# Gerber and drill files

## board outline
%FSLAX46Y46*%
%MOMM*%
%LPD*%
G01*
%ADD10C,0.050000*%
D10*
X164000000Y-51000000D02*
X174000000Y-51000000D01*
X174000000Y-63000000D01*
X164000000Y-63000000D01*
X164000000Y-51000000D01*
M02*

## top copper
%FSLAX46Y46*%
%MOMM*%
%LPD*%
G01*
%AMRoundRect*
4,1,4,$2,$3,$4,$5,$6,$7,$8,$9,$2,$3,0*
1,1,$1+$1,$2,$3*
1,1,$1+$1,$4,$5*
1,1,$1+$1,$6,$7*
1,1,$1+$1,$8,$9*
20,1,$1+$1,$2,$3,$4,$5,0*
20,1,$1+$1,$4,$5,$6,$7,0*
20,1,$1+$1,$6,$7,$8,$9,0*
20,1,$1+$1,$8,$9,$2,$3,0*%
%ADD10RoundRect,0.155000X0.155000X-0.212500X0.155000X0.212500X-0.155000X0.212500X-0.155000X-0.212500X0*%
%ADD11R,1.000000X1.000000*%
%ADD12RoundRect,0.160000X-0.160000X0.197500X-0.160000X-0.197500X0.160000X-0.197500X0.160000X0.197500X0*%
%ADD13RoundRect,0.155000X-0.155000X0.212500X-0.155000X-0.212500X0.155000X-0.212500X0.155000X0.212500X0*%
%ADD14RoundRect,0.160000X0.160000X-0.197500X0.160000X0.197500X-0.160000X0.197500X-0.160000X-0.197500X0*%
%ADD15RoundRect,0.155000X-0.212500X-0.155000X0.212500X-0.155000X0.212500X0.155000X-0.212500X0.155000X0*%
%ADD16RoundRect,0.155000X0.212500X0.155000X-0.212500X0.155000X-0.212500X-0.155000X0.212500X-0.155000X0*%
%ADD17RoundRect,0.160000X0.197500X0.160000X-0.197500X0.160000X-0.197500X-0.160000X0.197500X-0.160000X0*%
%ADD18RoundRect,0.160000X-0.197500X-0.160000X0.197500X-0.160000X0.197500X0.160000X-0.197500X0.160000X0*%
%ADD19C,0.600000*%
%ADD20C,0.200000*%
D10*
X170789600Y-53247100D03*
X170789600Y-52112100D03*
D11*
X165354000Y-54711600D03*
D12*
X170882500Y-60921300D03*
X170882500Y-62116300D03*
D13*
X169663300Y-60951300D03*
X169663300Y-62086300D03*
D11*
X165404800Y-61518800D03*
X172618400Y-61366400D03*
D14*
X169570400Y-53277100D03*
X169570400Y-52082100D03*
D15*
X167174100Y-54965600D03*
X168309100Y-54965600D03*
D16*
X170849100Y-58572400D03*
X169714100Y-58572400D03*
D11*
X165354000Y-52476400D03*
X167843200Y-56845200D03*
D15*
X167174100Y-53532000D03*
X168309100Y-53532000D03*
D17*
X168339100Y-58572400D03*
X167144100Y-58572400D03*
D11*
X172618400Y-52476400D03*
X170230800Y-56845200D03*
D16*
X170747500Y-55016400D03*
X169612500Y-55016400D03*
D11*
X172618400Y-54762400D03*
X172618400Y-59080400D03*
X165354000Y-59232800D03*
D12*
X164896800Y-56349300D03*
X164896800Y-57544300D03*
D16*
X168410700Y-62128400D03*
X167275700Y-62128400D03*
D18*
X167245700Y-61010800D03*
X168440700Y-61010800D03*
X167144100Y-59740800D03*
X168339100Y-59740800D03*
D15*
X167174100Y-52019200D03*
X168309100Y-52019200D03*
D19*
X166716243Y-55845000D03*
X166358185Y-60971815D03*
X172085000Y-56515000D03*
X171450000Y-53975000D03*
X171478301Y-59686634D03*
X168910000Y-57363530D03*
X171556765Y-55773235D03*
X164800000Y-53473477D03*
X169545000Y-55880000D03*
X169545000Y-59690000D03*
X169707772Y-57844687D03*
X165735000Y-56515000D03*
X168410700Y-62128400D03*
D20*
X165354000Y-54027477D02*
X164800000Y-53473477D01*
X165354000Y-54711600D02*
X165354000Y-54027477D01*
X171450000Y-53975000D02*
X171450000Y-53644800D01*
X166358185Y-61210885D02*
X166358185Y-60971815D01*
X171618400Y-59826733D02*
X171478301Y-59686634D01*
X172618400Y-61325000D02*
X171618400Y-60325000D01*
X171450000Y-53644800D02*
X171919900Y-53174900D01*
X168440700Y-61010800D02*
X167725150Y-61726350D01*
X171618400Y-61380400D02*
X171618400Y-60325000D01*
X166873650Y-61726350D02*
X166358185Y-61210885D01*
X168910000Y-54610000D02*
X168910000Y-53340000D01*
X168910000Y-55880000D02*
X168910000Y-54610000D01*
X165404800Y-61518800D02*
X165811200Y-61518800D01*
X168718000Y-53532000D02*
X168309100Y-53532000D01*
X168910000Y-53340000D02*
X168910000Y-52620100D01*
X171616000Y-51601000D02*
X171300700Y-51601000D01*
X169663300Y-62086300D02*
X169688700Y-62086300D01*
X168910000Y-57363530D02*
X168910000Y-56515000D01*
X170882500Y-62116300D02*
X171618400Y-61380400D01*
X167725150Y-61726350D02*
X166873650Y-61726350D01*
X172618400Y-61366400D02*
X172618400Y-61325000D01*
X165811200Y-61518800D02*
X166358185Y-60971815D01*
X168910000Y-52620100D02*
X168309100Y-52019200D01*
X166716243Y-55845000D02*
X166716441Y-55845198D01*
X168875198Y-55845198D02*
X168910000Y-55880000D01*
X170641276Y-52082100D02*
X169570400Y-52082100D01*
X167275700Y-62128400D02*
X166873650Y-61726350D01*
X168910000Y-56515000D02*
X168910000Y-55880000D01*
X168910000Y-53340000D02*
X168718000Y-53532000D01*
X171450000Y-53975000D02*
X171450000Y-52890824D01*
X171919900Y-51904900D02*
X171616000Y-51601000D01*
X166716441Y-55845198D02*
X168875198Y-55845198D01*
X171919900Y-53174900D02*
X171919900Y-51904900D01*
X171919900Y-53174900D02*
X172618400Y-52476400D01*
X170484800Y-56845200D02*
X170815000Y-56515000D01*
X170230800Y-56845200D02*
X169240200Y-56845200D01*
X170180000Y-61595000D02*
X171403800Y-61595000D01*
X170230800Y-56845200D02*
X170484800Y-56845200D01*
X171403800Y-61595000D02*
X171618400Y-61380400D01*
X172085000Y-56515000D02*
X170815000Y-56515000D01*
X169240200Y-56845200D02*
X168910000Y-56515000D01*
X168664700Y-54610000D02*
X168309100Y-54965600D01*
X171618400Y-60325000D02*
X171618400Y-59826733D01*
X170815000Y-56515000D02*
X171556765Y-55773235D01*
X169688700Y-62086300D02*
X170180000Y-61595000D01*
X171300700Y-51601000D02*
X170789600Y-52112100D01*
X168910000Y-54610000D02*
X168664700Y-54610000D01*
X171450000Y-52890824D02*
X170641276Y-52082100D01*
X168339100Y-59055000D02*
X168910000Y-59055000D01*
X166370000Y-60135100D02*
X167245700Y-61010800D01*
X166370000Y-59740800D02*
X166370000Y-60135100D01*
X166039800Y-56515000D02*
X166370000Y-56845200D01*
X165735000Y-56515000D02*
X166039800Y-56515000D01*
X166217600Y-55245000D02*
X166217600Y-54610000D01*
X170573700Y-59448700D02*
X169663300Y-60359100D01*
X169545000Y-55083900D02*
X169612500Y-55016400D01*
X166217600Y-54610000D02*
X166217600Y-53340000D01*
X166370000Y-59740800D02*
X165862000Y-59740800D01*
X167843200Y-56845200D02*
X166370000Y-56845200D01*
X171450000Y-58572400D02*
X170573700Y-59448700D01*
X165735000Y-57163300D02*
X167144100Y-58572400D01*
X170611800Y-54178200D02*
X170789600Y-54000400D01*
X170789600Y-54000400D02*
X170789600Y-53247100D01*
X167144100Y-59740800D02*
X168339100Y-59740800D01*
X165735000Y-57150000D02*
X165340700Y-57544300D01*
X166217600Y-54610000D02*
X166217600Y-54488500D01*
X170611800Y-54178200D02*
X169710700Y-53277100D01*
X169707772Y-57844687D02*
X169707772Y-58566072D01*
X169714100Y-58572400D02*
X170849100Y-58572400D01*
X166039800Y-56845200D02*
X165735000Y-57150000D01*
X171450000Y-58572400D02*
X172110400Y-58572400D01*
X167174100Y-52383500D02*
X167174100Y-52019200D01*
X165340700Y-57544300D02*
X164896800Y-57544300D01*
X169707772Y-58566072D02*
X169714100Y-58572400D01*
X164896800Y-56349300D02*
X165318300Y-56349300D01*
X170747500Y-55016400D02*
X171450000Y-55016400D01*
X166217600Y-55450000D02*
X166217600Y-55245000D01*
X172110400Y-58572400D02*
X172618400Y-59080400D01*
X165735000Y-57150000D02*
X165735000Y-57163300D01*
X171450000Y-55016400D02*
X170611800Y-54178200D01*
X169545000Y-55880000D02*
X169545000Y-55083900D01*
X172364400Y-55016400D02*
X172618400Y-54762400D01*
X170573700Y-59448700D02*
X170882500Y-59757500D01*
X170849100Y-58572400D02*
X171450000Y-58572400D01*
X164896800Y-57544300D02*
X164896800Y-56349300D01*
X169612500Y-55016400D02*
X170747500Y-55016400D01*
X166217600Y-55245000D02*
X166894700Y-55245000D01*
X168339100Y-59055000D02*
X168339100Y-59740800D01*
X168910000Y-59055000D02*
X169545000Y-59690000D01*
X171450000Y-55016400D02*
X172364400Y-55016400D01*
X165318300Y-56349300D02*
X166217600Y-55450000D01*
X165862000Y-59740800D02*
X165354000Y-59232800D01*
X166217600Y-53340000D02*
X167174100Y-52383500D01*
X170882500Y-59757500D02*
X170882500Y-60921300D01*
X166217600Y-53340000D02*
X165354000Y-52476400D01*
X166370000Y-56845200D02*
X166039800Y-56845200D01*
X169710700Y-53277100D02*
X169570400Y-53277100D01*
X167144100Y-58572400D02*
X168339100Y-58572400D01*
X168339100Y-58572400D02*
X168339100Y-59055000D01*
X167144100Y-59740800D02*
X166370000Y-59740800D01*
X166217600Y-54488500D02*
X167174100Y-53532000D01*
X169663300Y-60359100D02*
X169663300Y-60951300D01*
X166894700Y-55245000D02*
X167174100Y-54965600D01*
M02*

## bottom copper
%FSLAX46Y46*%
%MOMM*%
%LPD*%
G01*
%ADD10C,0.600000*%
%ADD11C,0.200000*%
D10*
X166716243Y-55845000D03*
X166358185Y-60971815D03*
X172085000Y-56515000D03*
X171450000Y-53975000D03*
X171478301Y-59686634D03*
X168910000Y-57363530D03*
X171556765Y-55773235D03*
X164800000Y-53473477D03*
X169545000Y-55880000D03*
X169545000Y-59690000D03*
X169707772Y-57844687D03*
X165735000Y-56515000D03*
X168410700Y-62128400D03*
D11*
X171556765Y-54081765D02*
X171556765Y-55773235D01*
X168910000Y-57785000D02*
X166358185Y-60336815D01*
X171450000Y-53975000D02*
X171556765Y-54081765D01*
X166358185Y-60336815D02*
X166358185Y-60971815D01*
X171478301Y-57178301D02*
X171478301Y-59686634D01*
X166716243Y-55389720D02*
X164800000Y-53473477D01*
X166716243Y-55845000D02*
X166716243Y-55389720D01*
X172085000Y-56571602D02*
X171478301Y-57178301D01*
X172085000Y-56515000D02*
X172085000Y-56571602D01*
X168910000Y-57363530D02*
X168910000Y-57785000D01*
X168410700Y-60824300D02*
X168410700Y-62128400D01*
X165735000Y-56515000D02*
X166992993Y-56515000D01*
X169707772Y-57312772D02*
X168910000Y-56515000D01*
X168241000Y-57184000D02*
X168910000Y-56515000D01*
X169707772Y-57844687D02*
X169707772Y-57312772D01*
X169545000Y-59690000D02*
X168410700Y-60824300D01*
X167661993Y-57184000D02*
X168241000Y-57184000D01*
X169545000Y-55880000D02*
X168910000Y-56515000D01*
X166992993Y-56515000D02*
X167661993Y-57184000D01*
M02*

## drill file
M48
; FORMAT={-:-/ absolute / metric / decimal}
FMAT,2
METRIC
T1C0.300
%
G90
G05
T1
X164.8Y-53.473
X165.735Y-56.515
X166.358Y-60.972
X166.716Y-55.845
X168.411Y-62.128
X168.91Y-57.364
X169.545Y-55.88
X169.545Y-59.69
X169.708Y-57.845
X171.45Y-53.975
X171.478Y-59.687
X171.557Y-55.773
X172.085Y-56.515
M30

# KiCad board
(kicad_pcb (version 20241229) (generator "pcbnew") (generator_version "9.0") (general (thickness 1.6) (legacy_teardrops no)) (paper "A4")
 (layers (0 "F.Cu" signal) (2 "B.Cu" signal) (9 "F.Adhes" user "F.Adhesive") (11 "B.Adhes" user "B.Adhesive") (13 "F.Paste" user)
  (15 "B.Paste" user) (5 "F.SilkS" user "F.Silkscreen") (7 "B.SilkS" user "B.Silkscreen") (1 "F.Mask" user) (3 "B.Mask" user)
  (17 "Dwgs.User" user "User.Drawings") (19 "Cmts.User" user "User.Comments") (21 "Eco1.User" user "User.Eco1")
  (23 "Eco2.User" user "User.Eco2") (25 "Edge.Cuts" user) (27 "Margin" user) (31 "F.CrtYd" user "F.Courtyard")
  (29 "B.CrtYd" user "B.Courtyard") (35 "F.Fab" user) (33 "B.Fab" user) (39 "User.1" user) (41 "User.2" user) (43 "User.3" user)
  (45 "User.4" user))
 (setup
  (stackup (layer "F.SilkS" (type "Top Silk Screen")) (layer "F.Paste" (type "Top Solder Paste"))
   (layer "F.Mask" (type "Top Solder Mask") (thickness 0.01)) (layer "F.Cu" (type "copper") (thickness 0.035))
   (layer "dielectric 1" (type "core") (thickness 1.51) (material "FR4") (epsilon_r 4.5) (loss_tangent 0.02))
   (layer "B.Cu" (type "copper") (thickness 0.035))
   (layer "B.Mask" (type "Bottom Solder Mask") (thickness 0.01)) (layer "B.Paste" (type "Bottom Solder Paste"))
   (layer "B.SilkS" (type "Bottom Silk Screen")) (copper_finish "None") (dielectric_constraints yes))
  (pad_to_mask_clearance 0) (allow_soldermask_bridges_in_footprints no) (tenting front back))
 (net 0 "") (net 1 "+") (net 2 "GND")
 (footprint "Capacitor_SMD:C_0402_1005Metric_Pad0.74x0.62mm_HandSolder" (layer "F.Cu") (at 170.7896 52.6796 90)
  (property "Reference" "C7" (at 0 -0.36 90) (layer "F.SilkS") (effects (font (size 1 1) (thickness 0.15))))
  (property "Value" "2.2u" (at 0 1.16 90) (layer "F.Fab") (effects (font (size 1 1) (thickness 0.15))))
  (pad "1" smd roundrect (at -0.5675 0 90) (size 0.735 0.62) (layers "F.Cu" "F.Mask" "F.Paste") (roundrect_rratio 0.25) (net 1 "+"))
  (pad "2" smd roundrect (at 0.5675 0 90) (size 0.735 0.62) (layers "F.Cu" "F.Mask" "F.Paste") (roundrect_rratio 0.25) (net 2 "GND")))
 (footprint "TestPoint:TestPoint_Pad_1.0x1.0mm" (layer "F.Cu") (at 165.354 54.7116)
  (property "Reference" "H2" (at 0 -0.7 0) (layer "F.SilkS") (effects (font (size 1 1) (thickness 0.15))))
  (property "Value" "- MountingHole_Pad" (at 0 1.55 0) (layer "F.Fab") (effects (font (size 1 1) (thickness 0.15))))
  (pad "1" smd rect (at 0 0) (size 1 1) (layers "F.Cu" "F.Mask")))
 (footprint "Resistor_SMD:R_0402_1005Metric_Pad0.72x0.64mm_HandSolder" (layer "F.Cu") (at 170.8825 61.5188 -90)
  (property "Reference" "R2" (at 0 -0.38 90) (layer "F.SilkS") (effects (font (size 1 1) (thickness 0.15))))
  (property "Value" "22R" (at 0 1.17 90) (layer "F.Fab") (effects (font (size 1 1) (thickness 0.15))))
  (pad "1" smd roundrect (at -0.5975 0 270) (size 0.715 0.64) (layers "F.Cu" "F.Mask" "F.Paste") (roundrect_rratio 0.25) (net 1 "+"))
  (pad "2" smd roundrect (at 0.5975 0 270) (size 0.715 0.64) (layers "F.Cu" "F.Mask" "F.Paste") (roundrect_rratio 0.25) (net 2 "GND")))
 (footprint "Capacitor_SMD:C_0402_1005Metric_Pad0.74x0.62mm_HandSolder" (layer "F.Cu") (at 169.6633 61.5188 -90)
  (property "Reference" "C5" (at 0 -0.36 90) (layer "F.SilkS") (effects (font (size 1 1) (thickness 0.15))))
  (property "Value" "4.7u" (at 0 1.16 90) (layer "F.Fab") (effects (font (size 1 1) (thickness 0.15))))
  (pad "1" smd roundrect (at -0.5675 0 270) (size 0.735 0.62) (layers "F.Cu" "F.Mask" "F.Paste") (roundrect_rratio 0.25) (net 1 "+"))
  (pad "2" smd roundrect (at 0.5675 0 270) (size 0.735 0.62) (layers "F.Cu" "F.Mask" "F.Paste") (roundrect_rratio 0.25) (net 2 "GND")))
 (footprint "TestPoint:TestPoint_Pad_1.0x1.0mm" (layer "F.Cu") (at 165.4048 61.5188)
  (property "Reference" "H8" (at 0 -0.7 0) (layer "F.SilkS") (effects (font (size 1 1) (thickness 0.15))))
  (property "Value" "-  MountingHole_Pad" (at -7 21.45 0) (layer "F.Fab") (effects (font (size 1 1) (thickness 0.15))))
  (pad "1" smd rect (at 0 0) (size 1 1) (layers "F.Cu" "F.Mask")))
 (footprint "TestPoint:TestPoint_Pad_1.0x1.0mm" (layer "F.Cu") (at 172.6184 61.3664)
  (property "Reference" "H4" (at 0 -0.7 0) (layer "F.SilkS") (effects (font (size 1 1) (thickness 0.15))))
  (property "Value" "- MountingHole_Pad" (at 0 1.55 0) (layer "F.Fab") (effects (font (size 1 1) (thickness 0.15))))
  (pad "1" smd rect (at 0 0) (size 1 1) (layers "F.Cu" "F.Mask")))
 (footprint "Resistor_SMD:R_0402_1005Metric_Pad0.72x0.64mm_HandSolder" (layer "F.Cu") (at 169.5704 52.6796 90)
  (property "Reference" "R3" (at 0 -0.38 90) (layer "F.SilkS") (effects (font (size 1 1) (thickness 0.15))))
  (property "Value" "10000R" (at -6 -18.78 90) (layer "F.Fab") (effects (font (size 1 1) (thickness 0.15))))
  (pad "1" smd roundrect (at -0.5975 0 90) (size 0.715 0.64) (layers "F.Cu" "F.Mask" "F.Paste") (roundrect_rratio 0.25) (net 1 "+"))
  (pad "2" smd roundrect (at 0.5975 0 90) (size 0.715 0.64) (layers "F.Cu" "F.Mask" "F.Paste") (roundrect_rratio 0.25) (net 2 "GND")))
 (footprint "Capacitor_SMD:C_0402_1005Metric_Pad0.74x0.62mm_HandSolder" (layer "F.Cu") (at 167.7416 54.9656)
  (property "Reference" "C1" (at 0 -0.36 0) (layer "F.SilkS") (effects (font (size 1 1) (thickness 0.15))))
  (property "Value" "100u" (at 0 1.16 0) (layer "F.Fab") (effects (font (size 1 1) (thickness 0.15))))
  (pad "1" smd roundrect (at -0.5675 0) (size 0.735 0.62) (layers "F.Cu" "F.Mask" "F.Paste") (roundrect_rratio 0.25) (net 1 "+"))
  (pad "2" smd roundrect (at 0.5675 0) (size 0.735 0.62) (layers "F.Cu" "F.Mask" "F.Paste") (roundrect_rratio 0.25) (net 2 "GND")))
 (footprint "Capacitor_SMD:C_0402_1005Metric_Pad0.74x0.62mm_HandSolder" (layer "F.Cu") (at 170.2816 58.5724 180)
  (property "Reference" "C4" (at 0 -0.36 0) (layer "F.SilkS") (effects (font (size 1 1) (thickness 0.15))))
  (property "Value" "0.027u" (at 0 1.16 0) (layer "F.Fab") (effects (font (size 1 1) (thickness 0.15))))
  (pad "1" smd roundrect (at -0.5675 0 180) (size 0.735 0.62) (layers "F.Cu" "F.Mask" "F.Paste") (roundrect_rratio 0.25) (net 1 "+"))
  (pad "2" smd roundrect (at 0.5675 0 180) (size 0.735 0.62) (layers "F.Cu" "F.Mask" "F.Paste") (roundrect_rratio 0.25) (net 1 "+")))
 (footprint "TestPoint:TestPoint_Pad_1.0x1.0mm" (layer "F.Cu") (at 165.354 52.4764)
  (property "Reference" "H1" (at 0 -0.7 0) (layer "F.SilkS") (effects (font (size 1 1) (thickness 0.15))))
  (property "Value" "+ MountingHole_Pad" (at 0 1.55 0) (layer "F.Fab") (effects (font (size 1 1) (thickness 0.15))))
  (pad "1" smd rect (at 0 0) (size 1 1) (layers "F.Cu" "F.Mask") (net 1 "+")))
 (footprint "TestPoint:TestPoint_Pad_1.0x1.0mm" (layer "F.Cu") (at 167.8432 56.8452)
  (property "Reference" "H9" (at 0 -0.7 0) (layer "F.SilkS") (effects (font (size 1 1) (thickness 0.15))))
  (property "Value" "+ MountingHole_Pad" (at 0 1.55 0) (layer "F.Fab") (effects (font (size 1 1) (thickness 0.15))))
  (pad "1" smd rect (at 0 0) (size 1 1) (layers "F.Cu" "F.Mask") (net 1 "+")))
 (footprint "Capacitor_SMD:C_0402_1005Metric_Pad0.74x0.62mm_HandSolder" (layer "F.Cu") (at 167.7416 53.532)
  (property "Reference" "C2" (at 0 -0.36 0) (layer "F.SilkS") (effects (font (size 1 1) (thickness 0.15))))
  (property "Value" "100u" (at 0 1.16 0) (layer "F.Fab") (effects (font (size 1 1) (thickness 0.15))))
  (pad "1" smd roundrect (at -0.5675 0) (size 0.735 0.62) (layers "F.Cu" "F.Mask" "F.Paste") (roundrect_rratio 0.25) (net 1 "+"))
  (pad "2" smd roundrect (at 0.5675 0) (size 0.735 0.62) (layers "F.Cu" "F.Mask" "F.Paste") (roundrect_rratio 0.25) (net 2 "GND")))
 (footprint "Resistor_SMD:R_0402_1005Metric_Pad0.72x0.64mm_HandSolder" (layer "F.Cu") (at 167.7416 58.5724 180)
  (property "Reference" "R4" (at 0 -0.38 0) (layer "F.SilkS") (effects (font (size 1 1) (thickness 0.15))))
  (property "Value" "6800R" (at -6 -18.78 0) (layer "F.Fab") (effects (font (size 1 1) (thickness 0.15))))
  (pad "1" smd roundrect (at -0.5975 0 180) (size 0.715 0.64) (layers "F.Cu" "F.Mask" "F.Paste") (roundrect_rratio 0.25) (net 1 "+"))
  (pad "2" smd roundrect (at 0.5975 0 180) (size 0.715 0.64) (layers "F.Cu" "F.Mask" "F.Paste") (roundrect_rratio 0.25) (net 1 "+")))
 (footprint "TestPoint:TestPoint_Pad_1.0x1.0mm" (layer "F.Cu") (at 172.6184 52.4764)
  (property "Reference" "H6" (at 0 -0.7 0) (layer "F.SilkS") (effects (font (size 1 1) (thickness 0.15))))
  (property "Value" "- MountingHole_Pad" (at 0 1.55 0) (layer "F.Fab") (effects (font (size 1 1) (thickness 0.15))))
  (pad "1" smd rect (at 0 0) (size 1 1) (layers "F.Cu" "F.Mask")))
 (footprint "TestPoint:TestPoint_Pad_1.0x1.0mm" (layer "F.Cu") (at 170.2308 56.8452)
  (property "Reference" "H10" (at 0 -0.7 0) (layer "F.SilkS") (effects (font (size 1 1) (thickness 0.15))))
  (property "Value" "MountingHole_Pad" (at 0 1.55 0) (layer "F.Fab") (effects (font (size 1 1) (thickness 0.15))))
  (pad "1" smd rect (at 0 0) (size 1 1) (layers "F.Cu" "F.Mask")))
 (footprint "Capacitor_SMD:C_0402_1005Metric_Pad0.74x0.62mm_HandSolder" (layer "F.Cu") (at 170.18 55.0164 180)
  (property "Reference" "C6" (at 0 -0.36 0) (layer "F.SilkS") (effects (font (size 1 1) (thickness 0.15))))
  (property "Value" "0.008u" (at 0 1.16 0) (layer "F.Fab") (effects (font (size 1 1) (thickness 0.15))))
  (pad "1" smd roundrect (at -0.5675 0 180) (size 0.735 0.62) (layers "F.Cu" "F.Mask" "F.Paste") (roundrect_rratio 0.25) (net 1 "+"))
  (pad "2" smd roundrect (at 0.5675 0 180) (size 0.735 0.62) (layers "F.Cu" "F.Mask" "F.Paste") (roundrect_rratio 0.25) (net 1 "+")))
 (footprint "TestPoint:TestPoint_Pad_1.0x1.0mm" (layer "F.Cu") (at 172.6184 54.7624)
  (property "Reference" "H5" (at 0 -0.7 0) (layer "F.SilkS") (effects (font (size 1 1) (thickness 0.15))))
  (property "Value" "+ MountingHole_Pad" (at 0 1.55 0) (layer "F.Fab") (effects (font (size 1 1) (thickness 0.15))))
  (pad "1" smd rect (at 0 0) (size 1 1) (layers "F.Cu" "F.Mask") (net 1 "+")))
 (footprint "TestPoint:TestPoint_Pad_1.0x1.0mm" (layer "F.Cu") (at 172.6184 59.0804)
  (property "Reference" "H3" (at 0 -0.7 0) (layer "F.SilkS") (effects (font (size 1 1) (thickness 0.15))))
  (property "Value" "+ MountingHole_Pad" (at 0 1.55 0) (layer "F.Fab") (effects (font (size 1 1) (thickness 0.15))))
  (pad "1" smd rect (at 0 0) (size 1 1) (layers "F.Cu" "F.Mask") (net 1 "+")))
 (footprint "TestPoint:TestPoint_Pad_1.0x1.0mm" (layer "F.Cu") (at 165.354 59.2328)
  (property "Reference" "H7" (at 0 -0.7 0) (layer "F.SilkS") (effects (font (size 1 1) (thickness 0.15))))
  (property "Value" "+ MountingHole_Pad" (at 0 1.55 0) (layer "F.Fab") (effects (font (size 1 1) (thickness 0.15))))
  (pad "1" smd rect (at 0 0) (size 1 1) (layers "F.Cu" "F.Mask") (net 1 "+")))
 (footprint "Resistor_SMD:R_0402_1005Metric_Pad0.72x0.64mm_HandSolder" (layer "F.Cu") (at 164.8968 56.9468 -90)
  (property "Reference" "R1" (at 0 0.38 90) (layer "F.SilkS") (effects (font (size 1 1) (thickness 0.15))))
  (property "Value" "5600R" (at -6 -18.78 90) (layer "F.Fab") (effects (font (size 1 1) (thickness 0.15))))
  (pad "1" smd roundrect (at -0.5975 0 270) (size 0.715 0.64) (layers "F.Cu" "F.Mask" "F.Paste") (roundrect_rratio 0.25) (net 1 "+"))
  (pad "2" smd roundrect (at 0.5975 0 270) (size 0.715 0.64) (layers "F.Cu" "F.Mask" "F.Paste") (roundrect_rratio 0.25) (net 1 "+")))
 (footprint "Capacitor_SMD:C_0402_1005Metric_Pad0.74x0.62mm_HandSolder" (layer "F.Cu") (at 167.8432 62.1284 180)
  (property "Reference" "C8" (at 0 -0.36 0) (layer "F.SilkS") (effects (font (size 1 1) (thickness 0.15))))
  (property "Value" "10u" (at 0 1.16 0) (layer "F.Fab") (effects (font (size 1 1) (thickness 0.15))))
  (pad "1" smd roundrect (at -0.5675 0 180) (size 0.735 0.62) (layers "F.Cu" "F.Mask" "F.Paste") (roundrect_rratio 0.25) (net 1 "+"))
  (pad "2" smd roundrect (at 0.5675 0 180) (size 0.735 0.62) (layers "F.Cu" "F.Mask" "F.Paste") (roundrect_rratio 0.25) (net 2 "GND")))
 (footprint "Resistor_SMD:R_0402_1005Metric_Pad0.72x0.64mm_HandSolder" (layer "F.Cu") (at 167.8432 61.0108)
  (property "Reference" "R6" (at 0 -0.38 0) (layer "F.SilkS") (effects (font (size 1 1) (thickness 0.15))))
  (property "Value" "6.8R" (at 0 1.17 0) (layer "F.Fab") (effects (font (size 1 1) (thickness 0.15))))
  (pad "1" smd roundrect (at -0.5975 0) (size 0.715 0.64) (layers "F.Cu" "F.Mask" "F.Paste") (roundrect_rratio 0.25) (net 1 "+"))
  (pad "2" smd roundrect (at 0.5975 0) (size 0.715 0.64) (layers "F.Cu" "F.Mask" "F.Paste") (roundrect_rratio 0.25) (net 2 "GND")))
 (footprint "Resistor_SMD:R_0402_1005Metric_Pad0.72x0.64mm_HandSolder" (layer "F.Cu") (at 167.7416 59.7408)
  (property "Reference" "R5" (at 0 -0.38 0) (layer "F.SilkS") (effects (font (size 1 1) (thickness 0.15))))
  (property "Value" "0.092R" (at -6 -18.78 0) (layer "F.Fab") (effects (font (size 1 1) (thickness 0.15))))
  (pad "1" smd roundrect (at -0.5975 0) (size 0.715 0.64) (layers "F.Cu" "F.Mask" "F.Paste") (roundrect_rratio 0.25) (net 1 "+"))
  (pad "2" smd roundrect (at 0.5975 0) (size 0.715 0.64) (layers "F.Cu" "F.Mask" "F.Paste") (roundrect_rratio 0.25) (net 1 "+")))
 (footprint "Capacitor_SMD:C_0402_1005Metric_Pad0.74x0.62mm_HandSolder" (layer "F.Cu") (at 167.7416 52.0192)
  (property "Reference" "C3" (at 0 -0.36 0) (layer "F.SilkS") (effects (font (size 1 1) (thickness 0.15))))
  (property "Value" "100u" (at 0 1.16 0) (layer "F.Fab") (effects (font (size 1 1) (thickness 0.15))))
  (pad "1" smd roundrect (at -0.5675 0) (size 0.735 0.62) (layers "F.Cu" "F.Mask" "F.Paste") (roundrect_rratio 0.25) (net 1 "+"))
  (pad "2" smd roundrect (at 0.5675 0) (size 0.735 0.62) (layers "F.Cu" "F.Mask" "F.Paste") (roundrect_rratio 0.25) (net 2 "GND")))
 (gr_rect (start 164 51) (end 174 63) (stroke (width 0.05) (type default)) (fill no) (layer "Edge.Cuts"))
 (segment (start 165.354 54.027477) (end 164.8 53.473477) (width 0.2) (layer "F.Cu") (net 2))
 (segment (start 165.354 54.7116) (end 165.354 54.027477) (width 0.2) (layer "F.Cu") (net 2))
 (segment (start 171.45 53.975) (end 171.45 53.6448) (width 0.2) (layer "F.Cu") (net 2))
 (segment (start 166.358185 61.210885) (end 166.358185 60.971815) (width 0.2) (layer "F.Cu") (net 2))
 (segment (start 171.6184 59.826733) (end 171.478301 59.686634) (width 0.2) (layer "F.Cu") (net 2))
 (segment (start 172.6184 61.325) (end 171.6184 60.325) (width 0.2) (layer "F.Cu") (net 2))
 (segment (start 171.45 53.6448) (end 171.9199 53.1749) (width 0.2) (layer "F.Cu") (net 2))
 (segment (start 168.4407 61.0108) (end 167.72515 61.72635) (width 0.2) (layer "F.Cu") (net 2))
 (segment (start 171.6184 61.3804) (end 171.6184 60.325) (width 0.2) (layer "F.Cu") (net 2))
 (segment (start 166.87365 61.72635) (end 166.358185 61.210885) (width 0.2) (layer "F.Cu") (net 2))
 (segment (start 168.91 54.61) (end 168.91 53.34) (width 0.2) (layer "F.Cu") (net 2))
 (segment (start 168.91 55.88) (end 168.91 54.61) (width 0.2) (layer "F.Cu") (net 2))
 (segment (start 165.4048 61.5188) (end 165.8112 61.5188) (width 0.2) (layer "F.Cu") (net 2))
 (segment (start 168.718 53.532) (end 168.3091 53.532) (width 0.2) (layer "F.Cu") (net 2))
 (segment (start 168.91 53.34) (end 168.91 52.6201) (width 0.2) (layer "F.Cu") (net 2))
 (segment (start 171.616 51.601) (end 171.3007 51.601) (width 0.2) (layer "F.Cu") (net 2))
 (segment (start 169.6633 62.0863) (end 169.6887 62.0863) (width 0.2) (layer "F.Cu") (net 2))
 (segment (start 168.91 57.36353) (end 168.91 56.515) (width 0.2) (layer "F.Cu") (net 2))
 (segment (start 170.8825 62.1163) (end 171.6184 61.3804) (width 0.2) (layer "F.Cu") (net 2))
 (segment (start 167.72515 61.72635) (end 166.87365 61.72635) (width 0.2) (layer "F.Cu") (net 2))
 (segment (start 172.6184 61.3664) (end 172.6184 61.325) (width 0.2) (layer "F.Cu") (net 2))
 (segment (start 165.8112 61.5188) (end 166.358185 60.971815) (width 0.2) (layer "F.Cu") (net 2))
 (segment (start 168.91 52.6201) (end 168.3091 52.0192) (width 0.2) (layer "F.Cu") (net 2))
 (segment (start 166.716243 55.845) (end 166.716441 55.845198) (width 0.2) (layer "F.Cu") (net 2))
 (segment (start 168.875198 55.845198) (end 168.91 55.88) (width 0.2) (layer "F.Cu") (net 2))
 (segment (start 170.641276 52.0821) (end 169.5704 52.0821) (width 0.2) (layer "F.Cu") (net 2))
 (segment (start 167.2757 62.1284) (end 166.87365 61.72635) (width 0.2) (layer "F.Cu") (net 2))
 (segment (start 168.91 56.515) (end 168.91 55.88) (width 0.2) (layer "F.Cu") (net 2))
 (segment (start 168.91 53.34) (end 168.718 53.532) (width 0.2) (layer "F.Cu") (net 2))
 (segment (start 171.45 53.975) (end 171.45 52.890824) (width 0.2) (layer "F.Cu") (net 2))
 (segment (start 171.9199 51.9049) (end 171.616 51.601) (width 0.2) (layer "F.Cu") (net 2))
 (segment (start 166.716441 55.845198) (end 168.875198 55.845198) (width 0.2) (layer "F.Cu") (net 2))
 (segment (start 171.9199 53.1749) (end 171.9199 51.9049) (width 0.2) (layer "F.Cu") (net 2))
 (segment (start 171.9199 53.1749) (end 172.6184 52.4764) (width 0.2) (layer "F.Cu") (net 2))
 (segment (start 170.4848 56.8452) (end 170.815 56.515) (width 0.2) (layer "F.Cu") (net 2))
 (segment (start 170.2308 56.8452) (end 169.2402 56.8452) (width 0.2) (layer "F.Cu") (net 2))
 (segment (start 170.18 61.595) (end 171.4038 61.595) (width 0.2) (layer "F.Cu") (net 2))
 (segment (start 170.2308 56.8452) (end 170.4848 56.8452) (width 0.2) (layer "F.Cu") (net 2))
 (segment (start 171.4038 61.595) (end 171.6184 61.3804) (width 0.2) (layer "F.Cu") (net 2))
 (segment (start 172.085 56.515) (end 170.815 56.515) (width 0.2) (layer "F.Cu") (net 2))
 (segment (start 169.2402 56.8452) (end 168.91 56.515) (width 0.2) (layer "F.Cu") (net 2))
 (segment (start 168.6647 54.61) (end 168.3091 54.9656) (width 0.2) (layer "F.Cu") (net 2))
 (segment (start 171.6184 60.325) (end 171.6184 59.826733) (width 0.2) (layer "F.Cu") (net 2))
 (segment (start 170.815 56.515) (end 171.556765 55.773235) (width 0.2) (layer "F.Cu") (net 2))
 (segment (start 169.6887 62.0863) (end 170.18 61.595) (width 0.2) (layer "F.Cu") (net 2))
 (segment (start 171.3007 51.601) (end 170.7896 52.1121) (width 0.2) (layer "F.Cu") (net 2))
 (segment (start 168.91 54.61) (end 168.6647 54.61) (width 0.2) (layer "F.Cu") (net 2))
 (segment (start 171.45 52.890824) (end 170.641276 52.0821) (width 0.2) (layer "F.Cu") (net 2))
 (via (at 166.716243 55.845) (size 0.6) (drill 0.3) (layers "F.Cu" "B.Cu") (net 2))
 (via (at 166.358185 60.971815) (size 0.6) (drill 0.3) (layers "F.Cu" "B.Cu") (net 2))
 (via (at 172.085 56.515) (size 0.6) (drill 0.3) (layers "F.Cu" "B.Cu") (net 2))
 (via (at 171.45 53.975) (size 0.6) (drill 0.3) (layers "F.Cu" "B.Cu") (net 2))
 (via (at 171.478301 59.686634) (size 0.6) (drill 0.3) (layers "F.Cu" "B.Cu") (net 2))
 (via (at 168.91 57.36353) (size 0.6) (drill 0.3) (layers "F.Cu" "B.Cu") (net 2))
 (via (at 171.556765 55.773235) (size 0.6) (drill 0.3) (layers "F.Cu" "B.Cu") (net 2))
 (via (at 164.8 53.473477) (size 0.6) (drill 0.3) (layers "F.Cu" "B.Cu") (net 2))
 (segment (start 171.556765 54.081765) (end 171.556765 55.773235) (width 0.2) (layer "B.Cu") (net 2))
 (segment (start 168.91 57.785) (end 166.358185 60.336815) (width 0.2) (layer "B.Cu") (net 2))
 (segment (start 171.45 53.975) (end 171.556765 54.081765) (width 0.2) (layer "B.Cu") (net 2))
 (segment (start 166.358185 60.336815) (end 166.358185 60.971815) (width 0.2) (layer "B.Cu") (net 2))
 (segment (start 171.478301 57.178301) (end 171.478301 59.686634) (width 0.2) (layer "B.Cu") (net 2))
 (segment (start 166.716243 55.38972) (end 164.8 53.473477) (width 0.2) (layer "B.Cu") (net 2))
 (segment (start 166.716243 55.845) (end 166.716243 55.38972) (width 0.2) (layer "B.Cu") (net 2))
 (segment (start 172.085 56.571602) (end 171.478301 57.178301) (width 0.2) (layer "B.Cu") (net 2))
 (segment (start 172.085 56.515) (end 172.085 56.571602) (width 0.2) (layer "B.Cu") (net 2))
 (segment (start 168.91 57.36353) (end 168.91 57.785) (width 0.2) (layer "B.Cu") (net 2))
 (segment (start 168.3391 59.055) (end 168.91 59.055) (width 0.2) (layer "F.Cu") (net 1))
 (segment (start 166.37 60.1351) (end 167.2457 61.0108) (width 0.2) (layer "F.Cu") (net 1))
 (segment (start 166.37 59.7408) (end 166.37 60.1351) (width 0.2) (layer "F.Cu") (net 1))
 (segment (start 166.0398 56.515) (end 166.37 56.8452) (width 0.2) (layer "F.Cu") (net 1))
 (segment (start 165.735 56.515) (end 166.0398 56.515) (width 0.2) (layer "F.Cu") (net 1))
 (segment (start 166.2176 55.245) (end 166.2176 54.61) (width 0.2) (layer "F.Cu") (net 1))
 (segment (start 170.5737 59.4487) (end 169.6633 60.3591) (width 0.2) (layer "F.Cu") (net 1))
 (segment (start 169.545 55.0839) (end 169.6125 55.0164) (width 0.2) (layer "F.Cu") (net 1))
 (segment (start 166.2176 54.61) (end 166.2176 53.34) (width 0.2) (layer "F.Cu") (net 1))
 (segment (start 166.37 59.7408) (end 165.862 59.7408) (width 0.2) (layer "F.Cu") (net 1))
 (segment (start 167.8432 56.8452) (end 166.37 56.8452) (width 0.2) (layer "F.Cu") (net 1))
 (segment (start 171.45 58.5724) (end 170.5737 59.4487) (width 0.2) (layer "F.Cu") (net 1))
 (segment (start 165.735 57.1633) (end 167.1441 58.5724) (width 0.2) (layer "F.Cu") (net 1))
 (segment (start 170.6118 54.1782) (end 170.7896 54.0004) (width 0.2) (layer "F.Cu") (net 1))
 (segment (start 170.7896 54.0004) (end 170.7896 53.2471) (width 0.2) (layer "F.Cu") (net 1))
 (segment (start 167.1441 59.7408) (end 168.3391 59.7408) (width 0.2) (layer "F.Cu") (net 1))
 (segment (start 165.735 57.15) (end 165.3407 57.5443) (width 0.2) (layer "F.Cu") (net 1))
 (segment (start 166.2176 54.61) (end 166.2176 54.4885) (width 0.2) (layer "F.Cu") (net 1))
 (segment (start 170.6118 54.1782) (end 169.7107 53.2771) (width 0.2) (layer "F.Cu") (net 1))
 (segment (start 169.707772 57.844687) (end 169.707772 58.566072) (width 0.2) (layer "F.Cu") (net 1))
 (segment (start 169.7141 58.5724) (end 170.8491 58.5724) (width 0.2) (layer "F.Cu") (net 1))
 (segment (start 166.0398 56.8452) (end 165.735 57.15) (width 0.2) (layer "F.Cu") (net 1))
 (segment (start 171.45 58.5724) (end 172.1104 58.5724) (width 0.2) (layer "F.Cu") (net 1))
 (segment (start 167.1741 52.3835) (end 167.1741 52.0192) (width 0.2) (layer "F.Cu") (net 1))
 (segment (start 165.3407 57.5443) (end 164.8968 57.5443) (width 0.2) (layer "F.Cu") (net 1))
 (segment (start 169.707772 58.566072) (end 169.7141 58.5724) (width 0.2) (layer "F.Cu") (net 1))
 (segment (start 164.8968 56.3493) (end 165.3183 56.3493) (width 0.2) (layer "F.Cu") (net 1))
 (segment (start 170.7475 55.0164) (end 171.45 55.0164) (width 0.2) (layer "F.Cu") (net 1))
 (segment (start 166.2176 55.45) (end 166.2176 55.245) (width 0.2) (layer "F.Cu") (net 1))
 (segment (start 172.1104 58.5724) (end 172.6184 59.0804) (width 0.2) (layer "F.Cu") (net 1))
 (segment (start 165.735 57.15) (end 165.735 57.1633) (width 0.2) (layer "F.Cu") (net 1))
 (segment (start 171.45 55.0164) (end 170.6118 54.1782) (width 0.2) (layer "F.Cu") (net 1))
 (segment (start 169.545 55.88) (end 169.545 55.0839) (width 0.2) (layer "F.Cu") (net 1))
 (segment (start 172.3644 55.0164) (end 172.6184 54.7624) (width 0.2) (layer "F.Cu") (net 1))
 (segment (start 170.5737 59.4487) (end 170.8825 59.7575) (width 0.2) (layer "F.Cu") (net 1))
 (segment (start 170.8491 58.5724) (end 171.45 58.5724) (width 0.2) (layer "F.Cu") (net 1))
 (segment (start 164.8968 57.5443) (end 164.8968 56.3493) (width 0.2) (layer "F.Cu") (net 1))
 (segment (start 169.6125 55.0164) (end 170.7475 55.0164) (width 0.2) (layer "F.Cu") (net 1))
 (segment (start 166.2176 55.245) (end 166.8947 55.245) (width 0.2) (layer "F.Cu") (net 1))
 (segment (start 168.3391 59.055) (end 168.3391 59.7408) (width 0.2) (layer "F.Cu") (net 1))
 (segment (start 168.91 59.055) (end 169.545 59.69) (width 0.2) (layer "F.Cu") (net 1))
 (segment (start 171.45 55.0164) (end 172.3644 55.0164) (width 0.2) (layer "F.Cu") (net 1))
 (segment (start 165.3183 56.3493) (end 166.2176 55.45) (width 0.2) (layer "F.Cu") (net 1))
 (segment (start 165.862 59.7408) (end 165.354 59.2328) (width 0.2) (layer "F.Cu") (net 1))
 (segment (start 166.2176 53.34) (end 167.1741 52.3835) (width 0.2) (layer "F.Cu") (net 1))
 (segment (start 170.8825 59.7575) (end 170.8825 60.9213) (width 0.2) (layer "F.Cu") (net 1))
 (segment (start 166.2176 53.34) (end 165.354 52.4764) (width 0.2) (layer "F.Cu") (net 1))
 (segment (start 166.37 56.8452) (end 166.0398 56.8452) (width 0.2) (layer "F.Cu") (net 1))
 (segment (start 169.7107 53.2771) (end 169.5704 53.2771) (width 0.2) (layer "F.Cu") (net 1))
 (segment (start 167.1441 58.5724) (end 168.3391 58.5724) (width 0.2) (layer "F.Cu") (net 1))
 (segment (start 168.3391 58.5724) (end 168.3391 59.055) (width 0.2) (layer "F.Cu") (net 1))
 (segment (start 167.1441 59.7408) (end 166.37 59.7408) (width 0.2) (layer "F.Cu") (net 1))
 (segment (start 166.2176 54.4885) (end 167.1741 53.532) (width 0.2) (layer "F.Cu") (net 1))
 (segment (start 169.6633 60.3591) (end 169.6633 60.9513) (width 0.2) (layer "F.Cu") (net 1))
 (segment (start 166.8947 55.245) (end 167.1741 54.9656) (width 0.2) (layer "F.Cu") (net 1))
 (via (at 169.545 55.88) (size 0.6) (drill 0.3) (layers "F.Cu" "B.Cu") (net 1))
 (via (at 169.545 59.69) (size 0.6) (drill 0.3) (layers "F.Cu" "B.Cu") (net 1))
 (via (at 169.707772 57.844687) (size 0.6) (drill 0.3) (layers "F.Cu" "B.Cu") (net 1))
 (via (at 165.735 56.515) (size 0.6) (drill 0.3) (layers "F.Cu" "B.Cu") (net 1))
 (via (at 168.4107 62.1284) (size 0.6) (drill 0.3) (layers "F.Cu" "B.Cu") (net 1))
 (segment (start 168.4107 60.8243) (end 168.4107 62.1284) (width 0.2) (layer "B.Cu") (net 1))
 (segment (start 165.735 56.515) (end 166.992993 56.515) (width 0.2) (layer "B.Cu") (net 1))
 (segment (start 169.707772 57.312772) (end 168.91 56.515) (width 0.2) (layer "B.Cu") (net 1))
 (segment (start 168.241 57.184) (end 168.91 56.515) (width 0.2) (layer "B.Cu") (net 1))
 (segment (start 169.707772 57.844687) (end 169.707772 57.312772) (width 0.2) (layer "B.Cu") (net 1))
 (segment (start 169.545 59.69) (end 168.4107 60.8243) (width 0.2) (layer "B.Cu") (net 1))
 (segment (start 167.661993 57.184) (end 168.241 57.184) (width 0.2) (layer "B.Cu") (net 1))
 (segment (start 169.545 55.88) (end 168.91 56.515) (width 0.2) (layer "B.Cu") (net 1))
 (segment (start 166.992993 56.515) (end 167.661993 57.184) (width 0.2) (layer "B.Cu") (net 1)))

